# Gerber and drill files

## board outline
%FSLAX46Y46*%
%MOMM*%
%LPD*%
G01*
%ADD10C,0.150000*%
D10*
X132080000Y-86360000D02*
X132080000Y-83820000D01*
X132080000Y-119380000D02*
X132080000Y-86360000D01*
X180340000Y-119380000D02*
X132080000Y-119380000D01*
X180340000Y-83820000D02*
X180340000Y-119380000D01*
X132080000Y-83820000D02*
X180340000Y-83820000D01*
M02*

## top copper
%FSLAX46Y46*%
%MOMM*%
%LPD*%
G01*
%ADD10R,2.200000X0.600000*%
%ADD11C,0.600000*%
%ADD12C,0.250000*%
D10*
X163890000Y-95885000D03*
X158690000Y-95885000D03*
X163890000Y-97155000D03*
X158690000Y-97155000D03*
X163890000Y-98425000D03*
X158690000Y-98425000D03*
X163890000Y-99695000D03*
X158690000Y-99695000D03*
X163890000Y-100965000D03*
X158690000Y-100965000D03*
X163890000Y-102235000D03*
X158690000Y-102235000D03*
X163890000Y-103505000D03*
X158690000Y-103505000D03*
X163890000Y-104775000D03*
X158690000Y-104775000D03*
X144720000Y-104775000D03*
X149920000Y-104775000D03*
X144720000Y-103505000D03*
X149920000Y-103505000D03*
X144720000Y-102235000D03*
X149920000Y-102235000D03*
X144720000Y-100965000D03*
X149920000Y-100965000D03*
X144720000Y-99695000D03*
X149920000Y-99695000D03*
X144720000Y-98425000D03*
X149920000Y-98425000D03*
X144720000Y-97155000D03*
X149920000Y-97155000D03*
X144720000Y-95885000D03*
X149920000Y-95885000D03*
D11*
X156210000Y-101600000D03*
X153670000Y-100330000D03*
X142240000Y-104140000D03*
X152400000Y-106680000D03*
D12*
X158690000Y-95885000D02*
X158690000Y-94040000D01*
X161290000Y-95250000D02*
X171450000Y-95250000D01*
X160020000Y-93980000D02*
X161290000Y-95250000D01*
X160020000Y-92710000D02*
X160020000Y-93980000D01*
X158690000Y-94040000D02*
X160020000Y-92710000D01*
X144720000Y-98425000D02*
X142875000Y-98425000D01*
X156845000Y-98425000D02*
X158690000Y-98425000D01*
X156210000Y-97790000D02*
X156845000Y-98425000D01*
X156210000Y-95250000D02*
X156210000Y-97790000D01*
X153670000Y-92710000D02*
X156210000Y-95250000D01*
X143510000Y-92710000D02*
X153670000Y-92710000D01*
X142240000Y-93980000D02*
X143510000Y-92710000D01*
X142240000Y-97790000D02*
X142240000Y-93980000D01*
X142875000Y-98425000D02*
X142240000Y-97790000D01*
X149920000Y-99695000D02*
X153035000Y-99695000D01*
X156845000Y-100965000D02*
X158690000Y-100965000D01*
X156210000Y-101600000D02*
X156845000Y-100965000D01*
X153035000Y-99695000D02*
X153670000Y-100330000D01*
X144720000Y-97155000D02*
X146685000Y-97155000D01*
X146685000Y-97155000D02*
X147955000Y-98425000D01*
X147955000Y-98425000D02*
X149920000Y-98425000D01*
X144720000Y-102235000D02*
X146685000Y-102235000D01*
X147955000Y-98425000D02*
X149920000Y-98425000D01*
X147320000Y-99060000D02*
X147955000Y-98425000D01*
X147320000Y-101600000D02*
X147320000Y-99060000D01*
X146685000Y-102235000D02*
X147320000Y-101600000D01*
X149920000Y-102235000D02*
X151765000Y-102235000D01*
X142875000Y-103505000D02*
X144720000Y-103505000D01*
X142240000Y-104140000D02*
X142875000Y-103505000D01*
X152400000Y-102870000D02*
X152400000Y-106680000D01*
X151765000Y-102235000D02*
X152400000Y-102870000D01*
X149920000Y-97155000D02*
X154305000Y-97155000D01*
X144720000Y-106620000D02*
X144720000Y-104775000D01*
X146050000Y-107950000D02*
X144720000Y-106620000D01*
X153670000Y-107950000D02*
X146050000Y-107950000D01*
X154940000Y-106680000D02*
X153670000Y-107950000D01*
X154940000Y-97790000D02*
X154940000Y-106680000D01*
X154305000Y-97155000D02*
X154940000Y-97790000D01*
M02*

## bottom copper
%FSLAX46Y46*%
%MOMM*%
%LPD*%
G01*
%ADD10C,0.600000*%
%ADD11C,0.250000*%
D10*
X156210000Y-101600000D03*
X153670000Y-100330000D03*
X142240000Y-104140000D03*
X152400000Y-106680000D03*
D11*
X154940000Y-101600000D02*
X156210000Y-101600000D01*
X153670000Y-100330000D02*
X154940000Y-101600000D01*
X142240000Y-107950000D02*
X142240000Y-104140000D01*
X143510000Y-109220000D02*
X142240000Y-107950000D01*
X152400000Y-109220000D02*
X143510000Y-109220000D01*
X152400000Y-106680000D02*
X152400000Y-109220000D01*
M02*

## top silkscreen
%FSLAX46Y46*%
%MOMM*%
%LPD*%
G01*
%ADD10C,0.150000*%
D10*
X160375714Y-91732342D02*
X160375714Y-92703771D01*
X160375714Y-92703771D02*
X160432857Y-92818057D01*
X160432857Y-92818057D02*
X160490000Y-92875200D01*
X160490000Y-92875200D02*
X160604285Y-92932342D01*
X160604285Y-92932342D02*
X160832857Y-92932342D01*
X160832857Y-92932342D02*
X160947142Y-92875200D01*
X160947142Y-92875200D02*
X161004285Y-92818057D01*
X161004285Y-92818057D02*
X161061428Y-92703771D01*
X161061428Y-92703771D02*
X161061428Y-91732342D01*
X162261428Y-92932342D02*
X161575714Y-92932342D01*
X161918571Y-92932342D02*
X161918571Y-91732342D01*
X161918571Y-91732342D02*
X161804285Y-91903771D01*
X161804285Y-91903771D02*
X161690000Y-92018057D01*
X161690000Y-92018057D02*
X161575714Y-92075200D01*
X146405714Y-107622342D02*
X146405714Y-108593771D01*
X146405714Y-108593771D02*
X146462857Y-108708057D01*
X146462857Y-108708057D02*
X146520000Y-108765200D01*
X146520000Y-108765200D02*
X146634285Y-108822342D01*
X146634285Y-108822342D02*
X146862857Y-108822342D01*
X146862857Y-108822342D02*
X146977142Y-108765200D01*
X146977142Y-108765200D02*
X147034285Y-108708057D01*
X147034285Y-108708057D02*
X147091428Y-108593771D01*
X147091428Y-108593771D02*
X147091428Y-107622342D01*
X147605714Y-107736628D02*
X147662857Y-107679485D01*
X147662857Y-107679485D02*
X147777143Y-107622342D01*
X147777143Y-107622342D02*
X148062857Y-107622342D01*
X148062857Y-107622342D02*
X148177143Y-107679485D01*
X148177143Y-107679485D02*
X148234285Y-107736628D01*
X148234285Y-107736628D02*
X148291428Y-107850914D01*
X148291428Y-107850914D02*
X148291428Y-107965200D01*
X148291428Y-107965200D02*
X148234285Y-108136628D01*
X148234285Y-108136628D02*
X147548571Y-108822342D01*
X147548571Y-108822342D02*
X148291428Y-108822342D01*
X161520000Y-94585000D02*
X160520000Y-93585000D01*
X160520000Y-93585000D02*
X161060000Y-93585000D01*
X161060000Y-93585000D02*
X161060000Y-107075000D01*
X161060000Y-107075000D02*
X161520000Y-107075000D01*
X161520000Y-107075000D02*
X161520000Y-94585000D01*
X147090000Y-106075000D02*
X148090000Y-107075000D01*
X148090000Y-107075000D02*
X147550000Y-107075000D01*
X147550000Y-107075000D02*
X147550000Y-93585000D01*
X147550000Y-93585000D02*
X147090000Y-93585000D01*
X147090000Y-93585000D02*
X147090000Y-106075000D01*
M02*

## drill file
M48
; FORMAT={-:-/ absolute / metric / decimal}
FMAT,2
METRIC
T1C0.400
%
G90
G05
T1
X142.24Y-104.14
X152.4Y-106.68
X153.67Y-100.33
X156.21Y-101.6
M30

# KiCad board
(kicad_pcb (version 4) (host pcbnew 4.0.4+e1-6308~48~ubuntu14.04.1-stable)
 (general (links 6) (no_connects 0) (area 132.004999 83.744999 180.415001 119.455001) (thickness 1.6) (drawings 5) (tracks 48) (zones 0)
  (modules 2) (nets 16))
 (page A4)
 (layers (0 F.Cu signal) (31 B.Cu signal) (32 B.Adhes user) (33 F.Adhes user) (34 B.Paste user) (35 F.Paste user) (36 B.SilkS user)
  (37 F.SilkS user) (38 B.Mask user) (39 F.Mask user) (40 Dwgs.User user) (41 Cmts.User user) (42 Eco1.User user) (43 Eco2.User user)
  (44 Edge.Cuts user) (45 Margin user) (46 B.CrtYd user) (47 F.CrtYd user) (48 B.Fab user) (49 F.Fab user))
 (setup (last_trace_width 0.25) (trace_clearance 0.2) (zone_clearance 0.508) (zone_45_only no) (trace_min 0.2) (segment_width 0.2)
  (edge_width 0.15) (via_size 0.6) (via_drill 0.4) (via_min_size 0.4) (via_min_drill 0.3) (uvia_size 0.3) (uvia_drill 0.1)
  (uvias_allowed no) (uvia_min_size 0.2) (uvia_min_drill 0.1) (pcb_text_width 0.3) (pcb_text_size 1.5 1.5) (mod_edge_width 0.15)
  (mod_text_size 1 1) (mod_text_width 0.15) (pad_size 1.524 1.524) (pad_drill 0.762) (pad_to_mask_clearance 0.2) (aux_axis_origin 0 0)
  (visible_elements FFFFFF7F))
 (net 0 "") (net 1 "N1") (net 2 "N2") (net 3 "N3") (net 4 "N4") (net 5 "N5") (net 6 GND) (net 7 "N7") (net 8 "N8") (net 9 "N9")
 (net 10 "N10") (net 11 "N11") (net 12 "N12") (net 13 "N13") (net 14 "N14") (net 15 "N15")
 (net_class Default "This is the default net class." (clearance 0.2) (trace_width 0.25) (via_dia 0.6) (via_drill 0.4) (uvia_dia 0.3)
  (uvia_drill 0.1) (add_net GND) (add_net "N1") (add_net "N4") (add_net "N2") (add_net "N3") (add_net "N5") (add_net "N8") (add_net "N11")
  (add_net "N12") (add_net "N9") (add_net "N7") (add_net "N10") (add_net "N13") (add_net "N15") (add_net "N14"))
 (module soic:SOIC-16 (layer F.Cu) (at 161.29 100.33 270)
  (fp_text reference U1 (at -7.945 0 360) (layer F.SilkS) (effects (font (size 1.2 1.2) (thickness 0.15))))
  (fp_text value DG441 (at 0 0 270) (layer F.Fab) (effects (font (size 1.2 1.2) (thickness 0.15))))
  (fp_line (start -5.745 -0.23) (end -6.745 0.77) (layer F.SilkS) (width 0.15))
  (fp_line (start -6.745 0.77) (end -6.745 0.23) (layer F.SilkS) (width 0.15))
  (fp_line (start -6.745 0.23) (end 6.745 0.23) (layer F.SilkS) (width 0.15))
  (fp_line (start 6.745 0.23) (end 6.745 -0.23) (layer F.SilkS) (width 0.15))
  (fp_line (start 6.745 -0.23) (end -5.745 -0.23) (layer F.SilkS) (width 0.15))
  (pad 16 smd rect (at -4.445 -2.6 270) (size 0.6 2.2) (layers F.Cu F.Paste F.Mask))
  (pad 1 smd rect (at -4.445 2.6 270) (size 0.6 2.2) (layers F.Cu F.Paste F.Mask) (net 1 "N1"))
  (pad 15 smd rect (at -3.175 -2.6 270) (size 0.6 2.2) (layers F.Cu F.Paste F.Mask))
  (pad 2 smd rect (at -3.175 2.6 270) (size 0.6 2.2) (layers F.Cu F.Paste F.Mask) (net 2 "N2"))
  (pad 14 smd rect (at -1.905 -2.6 270) (size 0.6 2.2) (layers F.Cu F.Paste F.Mask))
  (pad 3 smd rect (at -1.905 2.6 270) (size 0.6 2.2) (layers F.Cu F.Paste F.Mask) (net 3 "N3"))
  (pad 13 smd rect (at -0.635 -2.6 270) (size 0.6 2.2) (layers F.Cu F.Paste F.Mask) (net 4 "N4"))
  (pad 4 smd rect (at -0.635 2.6 270) (size 0.6 2.2) (layers F.Cu F.Paste F.Mask) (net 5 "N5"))
  (pad 12 smd rect (at 0.635 -2.6 270) (size 0.6 2.2) (layers F.Cu F.Paste F.Mask))
  (pad 5 smd rect (at 0.635 2.6 270) (size 0.6 2.2) (layers F.Cu F.Paste F.Mask) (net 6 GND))
  (pad 11 smd rect (at 1.905 -2.6 270) (size 0.6 2.2) (layers F.Cu F.Paste F.Mask))
  (pad 6 smd rect (at 1.905 2.6 270) (size 0.6 2.2) (layers F.Cu F.Paste F.Mask))
  (pad 10 smd rect (at 3.175 -2.6 270) (size 0.6 2.2) (layers F.Cu F.Paste F.Mask))
  (pad 7 smd rect (at 3.175 2.6 270) (size 0.6 2.2) (layers F.Cu F.Paste F.Mask))
  (pad 9 smd rect (at 4.445 -2.6 270) (size 0.6 2.2) (layers F.Cu F.Paste F.Mask))
  (pad 8 smd rect (at 4.445 2.6 270) (size 0.6 2.2) (layers F.Cu F.Paste F.Mask)))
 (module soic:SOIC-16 (layer F.Cu) (at 147.32 100.33 90)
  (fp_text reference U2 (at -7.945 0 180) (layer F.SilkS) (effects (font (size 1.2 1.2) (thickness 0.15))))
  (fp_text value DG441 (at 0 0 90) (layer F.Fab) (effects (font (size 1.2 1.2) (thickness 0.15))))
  (fp_line (start -5.745 -0.23) (end -6.745 0.77) (layer F.SilkS) (width 0.15))
  (fp_line (start -6.745 0.77) (end -6.745 0.23) (layer F.SilkS) (width 0.15))
  (fp_line (start -6.745 0.23) (end 6.745 0.23) (layer F.SilkS) (width 0.15))
  (fp_line (start 6.745 0.23) (end 6.745 -0.23) (layer F.SilkS) (width 0.15))
  (fp_line (start 6.745 -0.23) (end -5.745 -0.23) (layer F.SilkS) (width 0.15))
  (pad 16 smd rect (at -4.445 -2.6 90) (size 0.6 2.2) (layers F.Cu F.Paste F.Mask) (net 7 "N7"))
  (pad 1 smd rect (at -4.445 2.6 90) (size 0.6 2.2) (layers F.Cu F.Paste F.Mask) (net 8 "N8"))
  (pad 15 smd rect (at -3.175 -2.6 90) (size 0.6 2.2) (layers F.Cu F.Paste F.Mask) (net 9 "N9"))
  (pad 2 smd rect (at -3.175 2.6 90) (size 0.6 2.2) (layers F.Cu F.Paste F.Mask) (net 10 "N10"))
  (pad 14 smd rect (at -1.905 -2.6 90) (size 0.6 2.2) (layers F.Cu F.Paste F.Mask) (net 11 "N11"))
  (pad 3 smd rect (at -1.905 2.6 90) (size 0.6 2.2) (layers F.Cu F.Paste F.Mask) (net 9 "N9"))
  (pad 13 smd rect (at -0.635 -2.6 90) (size 0.6 2.2) (layers F.Cu F.Paste F.Mask) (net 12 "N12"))
  (pad 4 smd rect (at -0.635 2.6 90) (size 0.6 2.2) (layers F.Cu F.Paste F.Mask) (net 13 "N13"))
  (pad 12 smd rect (at 0.635 -2.6 90) (size 0.6 2.2) (layers F.Cu F.Paste F.Mask))
  (pad 5 smd rect (at 0.635 2.6 90) (size 0.6 2.2) (layers F.Cu F.Paste F.Mask) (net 6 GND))
  (pad 11 smd rect (at 1.905 -2.6 90) (size 0.6 2.2) (layers F.Cu F.Paste F.Mask) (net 3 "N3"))
  (pad 6 smd rect (at 1.905 2.6 90) (size 0.6 2.2) (layers F.Cu F.Paste F.Mask) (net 11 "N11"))
  (pad 10 smd rect (at 3.175 -2.6 90) (size 0.6 2.2) (layers F.Cu F.Paste F.Mask) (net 11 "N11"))
  (pad 7 smd rect (at 3.175 2.6 90) (size 0.6 2.2) (layers F.Cu F.Paste F.Mask) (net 7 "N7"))
  (pad 9 smd rect (at 4.445 -2.6 90) (size 0.6 2.2) (layers F.Cu F.Paste F.Mask) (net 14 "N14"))
  (pad 8 smd rect (at 4.445 2.6 90) (size 0.6 2.2) (layers F.Cu F.Paste F.Mask) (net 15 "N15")))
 (gr_line (start 132.08 86.36) (end 132.08 83.82) (angle 90) (layer Edge.Cuts) (width 0.15))
 (gr_line (start 132.08 119.38) (end 132.08 86.36) (angle 90) (layer Edge.Cuts) (width 0.15))
 (gr_line (start 180.34 119.38) (end 132.08 119.38) (angle 90) (layer Edge.Cuts) (width 0.15))
 (gr_line (start 180.34 83.82) (end 180.34 119.38) (angle 90) (layer Edge.Cuts) (width 0.15))
 (gr_line (start 132.08 83.82) (end 180.34 83.82) (angle 90) (layer Edge.Cuts) (width 0.15))
 (segment (start 158.69 95.885) (end 158.69 94.04) (width 0.25) (layer F.Cu) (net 1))
 (segment (start 161.29 95.25) (end 171.45 95.25) (width 0.25) (layer F.Cu) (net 1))
 (segment (start 160.02 93.98) (end 161.29 95.25) (width 0.25) (layer F.Cu) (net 1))
 (segment (start 160.02 92.71) (end 160.02 93.98) (width 0.25) (layer F.Cu) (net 1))
 (segment (start 158.69 94.04) (end 160.02 92.71) (width 0.25) (layer F.Cu) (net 1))
 (segment (start 144.72 98.425) (end 142.875 98.425) (width 0.25) (layer F.Cu) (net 3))
 (segment (start 156.845 98.425) (end 158.69 98.425) (width 0.25) (layer F.Cu) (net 3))
 (segment (start 156.21 97.79) (end 156.845 98.425) (width 0.25) (layer F.Cu) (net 3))
 (segment (start 156.21 95.25) (end 156.21 97.79) (width 0.25) (layer F.Cu) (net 3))
 (segment (start 153.67 92.71) (end 156.21 95.25) (width 0.25) (layer F.Cu) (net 3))
 (segment (start 143.51 92.71) (end 153.67 92.71) (width 0.25) (layer F.Cu) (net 3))
 (segment (start 142.24 93.98) (end 143.51 92.71) (width 0.25) (layer F.Cu) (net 3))
 (segment (start 142.24 97.79) (end 142.24 93.98) (width 0.25) (layer F.Cu) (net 3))
 (segment (start 142.875 98.425) (end 142.24 97.79) (width 0.25) (layer F.Cu) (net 3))
 (segment (start 149.92 99.695) (end 153.035 99.695) (width 0.25) (layer F.Cu) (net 6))
 (segment (start 156.845 100.965) (end 158.69 100.965) (width 0.25) (layer F.Cu) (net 6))
 (segment (start 156.21 101.6) (end 156.845 100.965) (width 0.25) (layer F.Cu) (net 6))
 (via (at 156.21 101.6) (size 0.6) (drill 0.4) (layers F.Cu B.Cu) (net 6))
 (segment (start 154.94 101.6) (end 156.21 101.6) (width 0.25) (layer B.Cu) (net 6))
 (segment (start 153.67 100.33) (end 154.94 101.6) (width 0.25) (layer B.Cu) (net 6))
 (via (at 153.67 100.33) (size 0.6) (drill 0.4) (layers F.Cu B.Cu) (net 6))
 (segment (start 153.035 99.695) (end 153.67 100.33) (width 0.25) (layer F.Cu) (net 6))
 (segment (start 144.72 97.155) (end 146.685 97.155) (width 0.25) (layer F.Cu) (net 11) (status 400000))
 (segment (start 146.685 97.155) (end 147.955 98.425) (width 0.25) (layer F.Cu) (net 11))
 (segment (start 147.955 98.425) (end 149.92 98.425) (width 0.25) (layer F.Cu) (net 11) (status 800000))
 (segment (start 144.72 102.235) (end 146.685 102.235) (width 0.25) (layer F.Cu) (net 11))
 (segment (start 147.955 98.425) (end 149.92 98.425) (width 0.25) (layer F.Cu) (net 11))
 (segment (start 147.32 99.06) (end 147.955 98.425) (width 0.25) (layer F.Cu) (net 11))
 (segment (start 147.32 101.6) (end 147.32 99.06) (width 0.25) (layer F.Cu) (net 11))
 (segment (start 146.685 102.235) (end 147.32 101.6) (width 0.25) (layer F.Cu) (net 11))
 (segment (start 149.92 102.235) (end 151.765 102.235) (width 0.25) (layer F.Cu) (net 9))
 (segment (start 142.875 103.505) (end 144.72 103.505) (width 0.25) (layer F.Cu) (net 9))
 (segment (start 142.24 104.14) (end 142.875 103.505) (width 0.25) (layer F.Cu) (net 9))
 (via (at 142.24 104.14) (size 0.6) (drill 0.4) (layers F.Cu B.Cu) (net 9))
 (segment (start 142.24 107.95) (end 142.24 104.14) (width 0.25) (layer B.Cu) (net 9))
 (segment (start 143.51 109.22) (end 142.24 107.95) (width 0.25) (layer B.Cu) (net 9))
 (segment (start 152.4 109.22) (end 143.51 109.22) (width 0.25) (layer B.Cu) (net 9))
 (segment (start 152.4 106.68) (end 152.4 109.22) (width 0.25) (layer B.Cu) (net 9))
 (via (at 152.4 106.68) (size 0.6) (drill 0.4) (layers F.Cu B.Cu) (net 9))
 (segment (start 152.4 102.87) (end 152.4 106.68) (width 0.25) (layer F.Cu) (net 9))
 (segment (start 151.765 102.235) (end 152.4 102.87) (width 0.25) (layer F.Cu) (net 9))
 (segment (start 149.92 97.155) (end 154.305 97.155) (width 0.25) (layer F.Cu) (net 7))
 (segment (start 144.72 106.62) (end 144.72 104.775) (width 0.25) (layer F.Cu) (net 7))
 (segment (start 146.05 107.95) (end 144.72 106.62) (width 0.25) (layer F.Cu) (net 7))
 (segment (start 153.67 107.95) (end 146.05 107.95) (width 0.25) (layer F.Cu) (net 7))
 (segment (start 154.94 106.68) (end 153.67 107.95) (width 0.25) (layer F.Cu) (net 7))
 (segment (start 154.94 97.79) (end 154.94 106.68) (width 0.25) (layer F.Cu) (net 7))
 (segment (start 154.305 97.155) (end 154.94 97.79) (width 0.25) (layer F.Cu) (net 7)))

